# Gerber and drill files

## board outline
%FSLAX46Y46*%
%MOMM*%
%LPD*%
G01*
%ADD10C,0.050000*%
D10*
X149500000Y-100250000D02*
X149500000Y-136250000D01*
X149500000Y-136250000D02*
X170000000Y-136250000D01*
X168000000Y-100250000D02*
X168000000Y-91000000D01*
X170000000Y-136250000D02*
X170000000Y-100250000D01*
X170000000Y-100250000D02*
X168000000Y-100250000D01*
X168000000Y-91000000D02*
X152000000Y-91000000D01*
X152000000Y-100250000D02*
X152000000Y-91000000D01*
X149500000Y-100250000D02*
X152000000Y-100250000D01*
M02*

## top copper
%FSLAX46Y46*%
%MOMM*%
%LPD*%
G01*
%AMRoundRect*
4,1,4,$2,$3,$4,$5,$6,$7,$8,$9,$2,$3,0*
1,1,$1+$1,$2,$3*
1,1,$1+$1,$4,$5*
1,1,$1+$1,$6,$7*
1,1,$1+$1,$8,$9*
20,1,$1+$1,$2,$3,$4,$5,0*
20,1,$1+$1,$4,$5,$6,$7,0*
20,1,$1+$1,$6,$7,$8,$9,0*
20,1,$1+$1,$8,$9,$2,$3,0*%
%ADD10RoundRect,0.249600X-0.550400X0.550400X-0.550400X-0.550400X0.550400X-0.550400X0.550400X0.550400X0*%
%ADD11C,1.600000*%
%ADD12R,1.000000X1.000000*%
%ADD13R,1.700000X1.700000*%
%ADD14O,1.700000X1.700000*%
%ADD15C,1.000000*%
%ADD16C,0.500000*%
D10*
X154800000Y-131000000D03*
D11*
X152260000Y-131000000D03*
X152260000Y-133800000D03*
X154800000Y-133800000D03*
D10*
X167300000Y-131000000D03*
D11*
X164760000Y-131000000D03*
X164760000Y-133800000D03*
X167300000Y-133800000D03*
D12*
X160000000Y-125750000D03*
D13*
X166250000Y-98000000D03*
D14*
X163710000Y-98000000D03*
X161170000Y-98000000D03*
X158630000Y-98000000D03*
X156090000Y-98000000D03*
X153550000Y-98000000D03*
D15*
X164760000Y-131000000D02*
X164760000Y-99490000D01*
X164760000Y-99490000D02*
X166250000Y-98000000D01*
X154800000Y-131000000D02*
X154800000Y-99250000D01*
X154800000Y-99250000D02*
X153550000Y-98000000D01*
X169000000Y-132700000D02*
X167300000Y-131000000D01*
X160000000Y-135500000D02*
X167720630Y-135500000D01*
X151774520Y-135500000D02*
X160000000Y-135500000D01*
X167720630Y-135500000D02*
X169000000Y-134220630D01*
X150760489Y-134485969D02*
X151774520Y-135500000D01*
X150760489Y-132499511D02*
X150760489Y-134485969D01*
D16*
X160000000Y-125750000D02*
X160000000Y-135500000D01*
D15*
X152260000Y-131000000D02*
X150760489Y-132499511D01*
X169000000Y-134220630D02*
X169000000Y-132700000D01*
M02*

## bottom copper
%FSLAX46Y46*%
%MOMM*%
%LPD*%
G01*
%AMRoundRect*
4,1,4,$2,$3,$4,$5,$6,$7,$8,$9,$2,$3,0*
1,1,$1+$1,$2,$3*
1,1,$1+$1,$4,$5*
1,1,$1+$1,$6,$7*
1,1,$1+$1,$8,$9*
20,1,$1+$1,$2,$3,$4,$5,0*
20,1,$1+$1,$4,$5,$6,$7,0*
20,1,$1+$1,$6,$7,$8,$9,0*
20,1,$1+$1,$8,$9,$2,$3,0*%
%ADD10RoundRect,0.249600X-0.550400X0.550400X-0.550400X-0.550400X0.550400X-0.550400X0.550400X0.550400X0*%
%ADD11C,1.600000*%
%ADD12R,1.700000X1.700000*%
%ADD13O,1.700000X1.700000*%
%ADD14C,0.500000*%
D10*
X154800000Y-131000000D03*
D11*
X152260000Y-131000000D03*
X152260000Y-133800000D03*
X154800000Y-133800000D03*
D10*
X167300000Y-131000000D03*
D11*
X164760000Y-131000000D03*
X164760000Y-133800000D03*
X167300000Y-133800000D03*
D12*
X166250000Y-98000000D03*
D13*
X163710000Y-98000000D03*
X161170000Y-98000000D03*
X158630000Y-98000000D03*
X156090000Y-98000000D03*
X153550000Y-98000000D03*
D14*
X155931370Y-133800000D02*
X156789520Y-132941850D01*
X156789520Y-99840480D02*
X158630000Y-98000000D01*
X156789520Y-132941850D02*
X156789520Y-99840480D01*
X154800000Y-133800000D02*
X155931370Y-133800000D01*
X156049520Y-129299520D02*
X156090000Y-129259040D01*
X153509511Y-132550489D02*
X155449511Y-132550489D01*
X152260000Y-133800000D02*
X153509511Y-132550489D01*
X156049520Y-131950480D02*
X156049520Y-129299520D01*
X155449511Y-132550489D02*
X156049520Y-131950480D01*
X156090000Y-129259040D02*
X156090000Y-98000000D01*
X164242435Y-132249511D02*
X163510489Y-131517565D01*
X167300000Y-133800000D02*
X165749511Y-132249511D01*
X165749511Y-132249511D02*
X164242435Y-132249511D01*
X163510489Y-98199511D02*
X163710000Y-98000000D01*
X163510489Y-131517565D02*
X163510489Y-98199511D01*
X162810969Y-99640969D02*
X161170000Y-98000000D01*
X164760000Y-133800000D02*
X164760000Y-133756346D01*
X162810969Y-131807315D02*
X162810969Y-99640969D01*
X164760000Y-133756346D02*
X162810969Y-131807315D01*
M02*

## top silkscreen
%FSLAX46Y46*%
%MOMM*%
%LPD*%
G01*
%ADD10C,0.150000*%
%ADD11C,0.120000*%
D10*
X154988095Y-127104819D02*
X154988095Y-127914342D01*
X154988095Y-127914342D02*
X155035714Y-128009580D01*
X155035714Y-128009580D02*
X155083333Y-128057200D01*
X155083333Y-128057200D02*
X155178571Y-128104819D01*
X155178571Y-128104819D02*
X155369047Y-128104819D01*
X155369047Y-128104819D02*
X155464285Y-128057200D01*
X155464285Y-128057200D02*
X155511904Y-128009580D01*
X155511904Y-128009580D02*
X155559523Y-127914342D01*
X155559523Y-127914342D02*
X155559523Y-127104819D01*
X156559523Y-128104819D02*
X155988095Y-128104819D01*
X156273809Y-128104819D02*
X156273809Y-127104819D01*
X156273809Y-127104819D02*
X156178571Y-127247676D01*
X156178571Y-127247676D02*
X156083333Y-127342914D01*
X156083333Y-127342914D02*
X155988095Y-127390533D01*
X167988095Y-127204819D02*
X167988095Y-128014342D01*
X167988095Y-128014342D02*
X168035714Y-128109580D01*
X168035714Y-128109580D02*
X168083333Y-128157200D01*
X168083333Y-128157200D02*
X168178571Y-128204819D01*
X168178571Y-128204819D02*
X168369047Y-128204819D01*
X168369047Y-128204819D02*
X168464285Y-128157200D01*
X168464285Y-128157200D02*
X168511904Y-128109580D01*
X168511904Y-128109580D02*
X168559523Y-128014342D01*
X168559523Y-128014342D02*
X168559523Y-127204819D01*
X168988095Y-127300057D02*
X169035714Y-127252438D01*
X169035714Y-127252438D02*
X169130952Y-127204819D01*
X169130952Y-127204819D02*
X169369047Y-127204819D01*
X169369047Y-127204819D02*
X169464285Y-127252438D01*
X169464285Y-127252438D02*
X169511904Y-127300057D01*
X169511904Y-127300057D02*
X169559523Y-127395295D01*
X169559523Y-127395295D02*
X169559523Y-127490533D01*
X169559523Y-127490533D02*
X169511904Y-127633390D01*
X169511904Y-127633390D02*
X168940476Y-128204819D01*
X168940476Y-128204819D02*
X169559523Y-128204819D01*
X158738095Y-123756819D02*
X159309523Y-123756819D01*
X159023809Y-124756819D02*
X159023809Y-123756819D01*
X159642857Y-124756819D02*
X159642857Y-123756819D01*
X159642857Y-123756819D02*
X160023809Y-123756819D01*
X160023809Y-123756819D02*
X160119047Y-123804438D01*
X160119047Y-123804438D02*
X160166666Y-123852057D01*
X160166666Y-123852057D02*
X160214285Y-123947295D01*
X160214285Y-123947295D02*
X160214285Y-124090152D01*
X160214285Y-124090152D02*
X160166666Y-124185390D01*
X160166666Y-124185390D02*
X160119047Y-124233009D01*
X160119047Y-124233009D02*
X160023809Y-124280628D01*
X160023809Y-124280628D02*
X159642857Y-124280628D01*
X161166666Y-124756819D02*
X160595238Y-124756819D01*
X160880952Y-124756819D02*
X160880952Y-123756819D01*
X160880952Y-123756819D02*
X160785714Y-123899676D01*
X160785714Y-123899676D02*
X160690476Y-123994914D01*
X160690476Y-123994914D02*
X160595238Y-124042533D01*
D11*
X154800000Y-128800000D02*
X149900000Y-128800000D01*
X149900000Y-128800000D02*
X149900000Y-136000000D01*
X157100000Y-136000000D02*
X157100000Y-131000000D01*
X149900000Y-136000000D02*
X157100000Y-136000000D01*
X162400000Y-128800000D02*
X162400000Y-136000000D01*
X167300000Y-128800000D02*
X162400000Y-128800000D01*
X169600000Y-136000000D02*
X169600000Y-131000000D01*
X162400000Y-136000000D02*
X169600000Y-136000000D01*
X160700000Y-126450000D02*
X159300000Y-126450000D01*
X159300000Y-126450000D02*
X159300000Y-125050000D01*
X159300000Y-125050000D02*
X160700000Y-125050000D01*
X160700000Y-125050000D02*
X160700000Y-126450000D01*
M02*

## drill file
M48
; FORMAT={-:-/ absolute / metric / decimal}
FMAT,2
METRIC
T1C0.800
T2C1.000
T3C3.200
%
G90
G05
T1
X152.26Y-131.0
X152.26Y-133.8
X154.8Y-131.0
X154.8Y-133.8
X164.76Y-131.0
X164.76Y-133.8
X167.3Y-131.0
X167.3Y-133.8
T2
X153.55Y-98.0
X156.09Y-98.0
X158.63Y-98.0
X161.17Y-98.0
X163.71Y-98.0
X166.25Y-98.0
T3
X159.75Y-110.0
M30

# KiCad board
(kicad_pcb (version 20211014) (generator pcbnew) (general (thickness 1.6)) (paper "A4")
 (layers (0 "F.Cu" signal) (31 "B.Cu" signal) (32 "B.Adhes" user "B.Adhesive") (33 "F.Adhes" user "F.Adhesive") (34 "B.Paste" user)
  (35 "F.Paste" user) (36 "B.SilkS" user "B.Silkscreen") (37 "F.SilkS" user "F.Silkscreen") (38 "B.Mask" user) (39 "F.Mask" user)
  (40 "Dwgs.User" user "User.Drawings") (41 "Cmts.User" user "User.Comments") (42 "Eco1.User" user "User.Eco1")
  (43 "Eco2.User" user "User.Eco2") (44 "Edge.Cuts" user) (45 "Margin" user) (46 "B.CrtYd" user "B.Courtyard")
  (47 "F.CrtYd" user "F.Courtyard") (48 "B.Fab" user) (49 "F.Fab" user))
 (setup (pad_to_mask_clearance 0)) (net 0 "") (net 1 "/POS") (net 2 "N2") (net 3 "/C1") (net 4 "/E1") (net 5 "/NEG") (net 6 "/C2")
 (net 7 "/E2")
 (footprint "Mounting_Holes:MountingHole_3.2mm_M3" (layer "F.Cu") (at 159.75 110)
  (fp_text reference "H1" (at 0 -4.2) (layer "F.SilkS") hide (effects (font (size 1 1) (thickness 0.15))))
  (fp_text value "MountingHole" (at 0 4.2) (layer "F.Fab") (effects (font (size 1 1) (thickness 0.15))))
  (pad "" np_thru_hole circle locked (at 0 0) (size 3.2 3.2) (drill 3.2) (layers *.Cu *.Mask)))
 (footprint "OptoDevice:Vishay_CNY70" (layer "F.Cu") (at 154.8 131 -90)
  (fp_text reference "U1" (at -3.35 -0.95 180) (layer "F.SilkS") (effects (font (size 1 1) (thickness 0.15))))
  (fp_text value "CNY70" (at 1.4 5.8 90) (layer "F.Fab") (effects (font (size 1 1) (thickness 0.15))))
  (fp_line (start -2.2 0) (end -2.2 4.9) (layer "F.SilkS") (width 0.12))
  (fp_line (start -2.2 4.9) (end 5 4.9) (layer "F.SilkS") (width 0.12))
  (fp_line (start 5 -2.3) (end 0 -2.3) (layer "F.SilkS") (width 0.12))
  (fp_line (start 5 4.9) (end 5 -2.3) (layer "F.SilkS") (width 0.12))
  (pad "1" thru_hole roundrect locked (at 0 0 270) (size 1.6 1.6) (drill 0.8) (layers *.Cu *.Mask) (roundrect_rratio 0.156) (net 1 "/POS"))
  (pad "2" thru_hole circle locked (at 0 2.54 270) (size 1.6 1.6) (drill 0.8) (layers *.Cu *.Mask) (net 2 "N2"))
  (pad "3" thru_hole circle locked (at 2.8 2.54 270) (size 1.6 1.6) (drill 0.8) (layers *.Cu *.Mask) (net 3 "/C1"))
  (pad "4" thru_hole circle locked (at 2.8 0 270) (size 1.6 1.6) (drill 0.8) (layers *.Cu *.Mask) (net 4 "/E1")))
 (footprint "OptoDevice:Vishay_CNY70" (layer "F.Cu") (at 167.3 131 -90)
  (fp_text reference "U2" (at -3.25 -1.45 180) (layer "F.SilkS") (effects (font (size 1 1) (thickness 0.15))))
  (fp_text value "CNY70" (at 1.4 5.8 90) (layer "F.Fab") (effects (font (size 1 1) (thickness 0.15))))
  (fp_line (start -2.2 4.9) (end 5 4.9) (layer "F.SilkS") (width 0.12))
  (fp_line (start -2.2 0) (end -2.2 4.9) (layer "F.SilkS") (width 0.12))
  (fp_line (start 5 -2.3) (end 0 -2.3) (layer "F.SilkS") (width 0.12))
  (fp_line (start 5 4.9) (end 5 -2.3) (layer "F.SilkS") (width 0.12))
  (pad "1" thru_hole roundrect locked (at 0 0 270) (size 1.6 1.6) (drill 0.8) (layers *.Cu *.Mask) (roundrect_rratio 0.156) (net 2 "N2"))
  (pad "2" thru_hole circle locked (at 0 2.54 270) (size 1.6 1.6) (drill 0.8) (layers *.Cu *.Mask) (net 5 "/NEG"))
  (pad "3" thru_hole circle locked (at 2.8 2.54 270) (size 1.6 1.6) (drill 0.8) (layers *.Cu *.Mask) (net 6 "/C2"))
  (pad "4" thru_hole circle locked (at 2.8 0 270) (size 1.6 1.6) (drill 0.8) (layers *.Cu *.Mask) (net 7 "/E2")))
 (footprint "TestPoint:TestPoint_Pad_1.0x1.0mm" (layer "F.Cu") (at 160 125.75)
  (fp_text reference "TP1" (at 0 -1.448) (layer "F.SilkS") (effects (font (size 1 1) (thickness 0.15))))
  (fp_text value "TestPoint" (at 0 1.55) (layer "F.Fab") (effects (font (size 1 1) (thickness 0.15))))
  (fp_line (start 0.7 0.7) (end -0.7 0.7) (layer "F.SilkS") (width 0.12))
  (fp_line (start -0.7 0.7) (end -0.7 -0.7) (layer "F.SilkS") (width 0.12))
  (fp_line (start -0.7 -0.7) (end 0.7 -0.7) (layer "F.SilkS") (width 0.12))
  (fp_line (start 0.7 -0.7) (end 0.7 0.7) (layer "F.SilkS") (width 0.12))
  (pad "1" smd rect locked (at 0 0) (size 1 1) (layers "F.Cu" "F.Mask") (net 2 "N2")))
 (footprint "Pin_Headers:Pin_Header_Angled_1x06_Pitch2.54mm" (layer "B.Cu") (at 166.25 98 90)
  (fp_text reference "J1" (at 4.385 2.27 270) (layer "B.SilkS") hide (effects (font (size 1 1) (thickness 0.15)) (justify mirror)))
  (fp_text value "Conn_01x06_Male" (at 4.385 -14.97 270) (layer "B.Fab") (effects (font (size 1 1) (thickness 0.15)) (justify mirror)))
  (pad "1" thru_hole rect (at 0 0 90) (size 1.7 1.7) (drill 1) (layers *.Cu *.Mask) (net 5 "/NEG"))
  (pad "2" thru_hole oval (at 0 -2.54 90) (size 1.7 1.7) (drill 1) (layers *.Cu *.Mask) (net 7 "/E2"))
  (pad "3" thru_hole oval (at 0 -5.08 90) (size 1.7 1.7) (drill 1) (layers *.Cu *.Mask) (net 6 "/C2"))
  (pad "4" thru_hole oval (at 0 -7.62 90) (size 1.7 1.7) (drill 1) (layers *.Cu *.Mask) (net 4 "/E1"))
  (pad "5" thru_hole oval (at 0 -10.16 90) (size 1.7 1.7) (drill 1) (layers *.Cu *.Mask) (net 3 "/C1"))
  (pad "6" thru_hole oval (at 0 -12.7 90) (size 1.7 1.7) (drill 1) (layers *.Cu *.Mask) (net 1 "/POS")))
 (gr_line (start 149.5 100.25) (end 149.5 136.25) (layer "Edge.Cuts") (width 0.05))
 (gr_line (start 149.5 136.25) (end 170 136.25) (layer "Edge.Cuts") (width 0.05))
 (gr_line (start 168 100.25) (end 168 91) (layer "Edge.Cuts") (width 0.05))
 (gr_line (start 170 136.25) (end 170 100.25) (layer "Edge.Cuts") (width 0.05))
 (gr_line (start 170 100.25) (end 168 100.25) (layer "Edge.Cuts") (width 0.05))
 (gr_line (start 168 91) (end 152 91) (layer "Edge.Cuts") (width 0.05))
 (gr_line (start 152 100.25) (end 152 91) (layer "Edge.Cuts") (width 0.05))
 (gr_line (start 149.5 100.25) (end 152 100.25) (layer "Edge.Cuts") (width 0.05))
 (segment (start 164.76 131) (end 164.76 99.49) (width 1) (layer "F.Cu") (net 5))
 (segment (start 164.76 99.49) (end 166.25 98) (width 1) (layer "F.Cu") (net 5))
 (segment (start 155.93137 133.8) (end 156.78952 132.94185) (width 0.5) (layer "B.Cu") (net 4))
 (segment (start 156.78952 99.84048) (end 158.63 98) (width 0.5) (layer "B.Cu") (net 4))
 (segment (start 156.78952 132.94185) (end 156.78952 99.84048) (width 0.5) (layer "B.Cu") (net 4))
 (segment (start 154.8 133.8) (end 155.93137 133.8) (width 0.5) (layer "B.Cu") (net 4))
 (segment (start 156.04952 129.29952) (end 156.09 129.25904) (width 0.5) (layer "B.Cu") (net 3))
 (segment (start 153.509511 132.550489) (end 155.449511 132.550489) (width 0.5) (layer "B.Cu") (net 3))
 (segment (start 152.26 133.8) (end 153.509511 132.550489) (width 0.5) (layer "B.Cu") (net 3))
 (segment (start 156.04952 131.95048) (end 156.04952 129.29952) (width 0.5) (layer "B.Cu") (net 3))
 (segment (start 155.449511 132.550489) (end 156.04952 131.95048) (width 0.5) (layer "B.Cu") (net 3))
 (segment (start 156.09 129.25904) (end 156.09 98) (width 0.5) (layer "B.Cu") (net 3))
 (segment (start 154.8 131) (end 154.8 99.25) (width 1) (layer "F.Cu") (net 1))
 (segment (start 154.8 99.25) (end 153.55 98) (width 1) (layer "F.Cu") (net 1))
 (segment (start 169 132.7) (end 167.3 131) (width 1) (layer "F.Cu") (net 2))
 (segment (start 160 135.5) (end 167.72063 135.5) (width 1) (layer "F.Cu") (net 2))
 (segment (start 151.77452 135.5) (end 160 135.5) (width 1) (layer "F.Cu") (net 2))
 (segment (start 167.72063 135.5) (end 169 134.22063) (width 1) (layer "F.Cu") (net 2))
 (segment (start 150.760489 134.485969) (end 151.77452 135.5) (width 1) (layer "F.Cu") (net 2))
 (segment (start 150.760489 132.499511) (end 150.760489 134.485969) (width 1) (layer "F.Cu") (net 2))
 (segment (start 160 125.75) (end 160 135.5) (width 0.5) (layer "F.Cu") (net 2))
 (segment (start 152.26 131) (end 150.760489 132.499511) (width 1) (layer "F.Cu") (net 2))
 (segment (start 169 134.22063) (end 169 132.7) (width 1) (layer "F.Cu") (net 2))
 (segment (start 164.242435 132.249511) (end 163.510489 131.517565) (width 0.5) (layer "B.Cu") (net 7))
 (segment (start 167.3 133.8) (end 165.749511 132.249511) (width 0.5) (layer "B.Cu") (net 7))
 (segment (start 165.749511 132.249511) (end 164.242435 132.249511) (width 0.5) (layer "B.Cu") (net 7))
 (segment (start 163.510489 98.199511) (end 163.71 98) (width 0.5) (layer "B.Cu") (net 7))
 (segment (start 163.510489 131.517565) (end 163.510489 98.199511) (width 0.5) (layer "B.Cu") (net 7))
 (segment (start 162.810969 99.640969) (end 161.17 98) (width 0.5) (layer "B.Cu") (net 6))
 (segment (start 164.76 133.8) (end 164.76 133.756346) (width 0.5) (layer "B.Cu") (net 6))
 (segment (start 162.810969 131.807315) (end 162.810969 99.640969) (width 0.5) (layer "B.Cu") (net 6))
 (segment (start 164.76 133.756346) (end 162.810969 131.807315) (width 0.5) (layer "B.Cu") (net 6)))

